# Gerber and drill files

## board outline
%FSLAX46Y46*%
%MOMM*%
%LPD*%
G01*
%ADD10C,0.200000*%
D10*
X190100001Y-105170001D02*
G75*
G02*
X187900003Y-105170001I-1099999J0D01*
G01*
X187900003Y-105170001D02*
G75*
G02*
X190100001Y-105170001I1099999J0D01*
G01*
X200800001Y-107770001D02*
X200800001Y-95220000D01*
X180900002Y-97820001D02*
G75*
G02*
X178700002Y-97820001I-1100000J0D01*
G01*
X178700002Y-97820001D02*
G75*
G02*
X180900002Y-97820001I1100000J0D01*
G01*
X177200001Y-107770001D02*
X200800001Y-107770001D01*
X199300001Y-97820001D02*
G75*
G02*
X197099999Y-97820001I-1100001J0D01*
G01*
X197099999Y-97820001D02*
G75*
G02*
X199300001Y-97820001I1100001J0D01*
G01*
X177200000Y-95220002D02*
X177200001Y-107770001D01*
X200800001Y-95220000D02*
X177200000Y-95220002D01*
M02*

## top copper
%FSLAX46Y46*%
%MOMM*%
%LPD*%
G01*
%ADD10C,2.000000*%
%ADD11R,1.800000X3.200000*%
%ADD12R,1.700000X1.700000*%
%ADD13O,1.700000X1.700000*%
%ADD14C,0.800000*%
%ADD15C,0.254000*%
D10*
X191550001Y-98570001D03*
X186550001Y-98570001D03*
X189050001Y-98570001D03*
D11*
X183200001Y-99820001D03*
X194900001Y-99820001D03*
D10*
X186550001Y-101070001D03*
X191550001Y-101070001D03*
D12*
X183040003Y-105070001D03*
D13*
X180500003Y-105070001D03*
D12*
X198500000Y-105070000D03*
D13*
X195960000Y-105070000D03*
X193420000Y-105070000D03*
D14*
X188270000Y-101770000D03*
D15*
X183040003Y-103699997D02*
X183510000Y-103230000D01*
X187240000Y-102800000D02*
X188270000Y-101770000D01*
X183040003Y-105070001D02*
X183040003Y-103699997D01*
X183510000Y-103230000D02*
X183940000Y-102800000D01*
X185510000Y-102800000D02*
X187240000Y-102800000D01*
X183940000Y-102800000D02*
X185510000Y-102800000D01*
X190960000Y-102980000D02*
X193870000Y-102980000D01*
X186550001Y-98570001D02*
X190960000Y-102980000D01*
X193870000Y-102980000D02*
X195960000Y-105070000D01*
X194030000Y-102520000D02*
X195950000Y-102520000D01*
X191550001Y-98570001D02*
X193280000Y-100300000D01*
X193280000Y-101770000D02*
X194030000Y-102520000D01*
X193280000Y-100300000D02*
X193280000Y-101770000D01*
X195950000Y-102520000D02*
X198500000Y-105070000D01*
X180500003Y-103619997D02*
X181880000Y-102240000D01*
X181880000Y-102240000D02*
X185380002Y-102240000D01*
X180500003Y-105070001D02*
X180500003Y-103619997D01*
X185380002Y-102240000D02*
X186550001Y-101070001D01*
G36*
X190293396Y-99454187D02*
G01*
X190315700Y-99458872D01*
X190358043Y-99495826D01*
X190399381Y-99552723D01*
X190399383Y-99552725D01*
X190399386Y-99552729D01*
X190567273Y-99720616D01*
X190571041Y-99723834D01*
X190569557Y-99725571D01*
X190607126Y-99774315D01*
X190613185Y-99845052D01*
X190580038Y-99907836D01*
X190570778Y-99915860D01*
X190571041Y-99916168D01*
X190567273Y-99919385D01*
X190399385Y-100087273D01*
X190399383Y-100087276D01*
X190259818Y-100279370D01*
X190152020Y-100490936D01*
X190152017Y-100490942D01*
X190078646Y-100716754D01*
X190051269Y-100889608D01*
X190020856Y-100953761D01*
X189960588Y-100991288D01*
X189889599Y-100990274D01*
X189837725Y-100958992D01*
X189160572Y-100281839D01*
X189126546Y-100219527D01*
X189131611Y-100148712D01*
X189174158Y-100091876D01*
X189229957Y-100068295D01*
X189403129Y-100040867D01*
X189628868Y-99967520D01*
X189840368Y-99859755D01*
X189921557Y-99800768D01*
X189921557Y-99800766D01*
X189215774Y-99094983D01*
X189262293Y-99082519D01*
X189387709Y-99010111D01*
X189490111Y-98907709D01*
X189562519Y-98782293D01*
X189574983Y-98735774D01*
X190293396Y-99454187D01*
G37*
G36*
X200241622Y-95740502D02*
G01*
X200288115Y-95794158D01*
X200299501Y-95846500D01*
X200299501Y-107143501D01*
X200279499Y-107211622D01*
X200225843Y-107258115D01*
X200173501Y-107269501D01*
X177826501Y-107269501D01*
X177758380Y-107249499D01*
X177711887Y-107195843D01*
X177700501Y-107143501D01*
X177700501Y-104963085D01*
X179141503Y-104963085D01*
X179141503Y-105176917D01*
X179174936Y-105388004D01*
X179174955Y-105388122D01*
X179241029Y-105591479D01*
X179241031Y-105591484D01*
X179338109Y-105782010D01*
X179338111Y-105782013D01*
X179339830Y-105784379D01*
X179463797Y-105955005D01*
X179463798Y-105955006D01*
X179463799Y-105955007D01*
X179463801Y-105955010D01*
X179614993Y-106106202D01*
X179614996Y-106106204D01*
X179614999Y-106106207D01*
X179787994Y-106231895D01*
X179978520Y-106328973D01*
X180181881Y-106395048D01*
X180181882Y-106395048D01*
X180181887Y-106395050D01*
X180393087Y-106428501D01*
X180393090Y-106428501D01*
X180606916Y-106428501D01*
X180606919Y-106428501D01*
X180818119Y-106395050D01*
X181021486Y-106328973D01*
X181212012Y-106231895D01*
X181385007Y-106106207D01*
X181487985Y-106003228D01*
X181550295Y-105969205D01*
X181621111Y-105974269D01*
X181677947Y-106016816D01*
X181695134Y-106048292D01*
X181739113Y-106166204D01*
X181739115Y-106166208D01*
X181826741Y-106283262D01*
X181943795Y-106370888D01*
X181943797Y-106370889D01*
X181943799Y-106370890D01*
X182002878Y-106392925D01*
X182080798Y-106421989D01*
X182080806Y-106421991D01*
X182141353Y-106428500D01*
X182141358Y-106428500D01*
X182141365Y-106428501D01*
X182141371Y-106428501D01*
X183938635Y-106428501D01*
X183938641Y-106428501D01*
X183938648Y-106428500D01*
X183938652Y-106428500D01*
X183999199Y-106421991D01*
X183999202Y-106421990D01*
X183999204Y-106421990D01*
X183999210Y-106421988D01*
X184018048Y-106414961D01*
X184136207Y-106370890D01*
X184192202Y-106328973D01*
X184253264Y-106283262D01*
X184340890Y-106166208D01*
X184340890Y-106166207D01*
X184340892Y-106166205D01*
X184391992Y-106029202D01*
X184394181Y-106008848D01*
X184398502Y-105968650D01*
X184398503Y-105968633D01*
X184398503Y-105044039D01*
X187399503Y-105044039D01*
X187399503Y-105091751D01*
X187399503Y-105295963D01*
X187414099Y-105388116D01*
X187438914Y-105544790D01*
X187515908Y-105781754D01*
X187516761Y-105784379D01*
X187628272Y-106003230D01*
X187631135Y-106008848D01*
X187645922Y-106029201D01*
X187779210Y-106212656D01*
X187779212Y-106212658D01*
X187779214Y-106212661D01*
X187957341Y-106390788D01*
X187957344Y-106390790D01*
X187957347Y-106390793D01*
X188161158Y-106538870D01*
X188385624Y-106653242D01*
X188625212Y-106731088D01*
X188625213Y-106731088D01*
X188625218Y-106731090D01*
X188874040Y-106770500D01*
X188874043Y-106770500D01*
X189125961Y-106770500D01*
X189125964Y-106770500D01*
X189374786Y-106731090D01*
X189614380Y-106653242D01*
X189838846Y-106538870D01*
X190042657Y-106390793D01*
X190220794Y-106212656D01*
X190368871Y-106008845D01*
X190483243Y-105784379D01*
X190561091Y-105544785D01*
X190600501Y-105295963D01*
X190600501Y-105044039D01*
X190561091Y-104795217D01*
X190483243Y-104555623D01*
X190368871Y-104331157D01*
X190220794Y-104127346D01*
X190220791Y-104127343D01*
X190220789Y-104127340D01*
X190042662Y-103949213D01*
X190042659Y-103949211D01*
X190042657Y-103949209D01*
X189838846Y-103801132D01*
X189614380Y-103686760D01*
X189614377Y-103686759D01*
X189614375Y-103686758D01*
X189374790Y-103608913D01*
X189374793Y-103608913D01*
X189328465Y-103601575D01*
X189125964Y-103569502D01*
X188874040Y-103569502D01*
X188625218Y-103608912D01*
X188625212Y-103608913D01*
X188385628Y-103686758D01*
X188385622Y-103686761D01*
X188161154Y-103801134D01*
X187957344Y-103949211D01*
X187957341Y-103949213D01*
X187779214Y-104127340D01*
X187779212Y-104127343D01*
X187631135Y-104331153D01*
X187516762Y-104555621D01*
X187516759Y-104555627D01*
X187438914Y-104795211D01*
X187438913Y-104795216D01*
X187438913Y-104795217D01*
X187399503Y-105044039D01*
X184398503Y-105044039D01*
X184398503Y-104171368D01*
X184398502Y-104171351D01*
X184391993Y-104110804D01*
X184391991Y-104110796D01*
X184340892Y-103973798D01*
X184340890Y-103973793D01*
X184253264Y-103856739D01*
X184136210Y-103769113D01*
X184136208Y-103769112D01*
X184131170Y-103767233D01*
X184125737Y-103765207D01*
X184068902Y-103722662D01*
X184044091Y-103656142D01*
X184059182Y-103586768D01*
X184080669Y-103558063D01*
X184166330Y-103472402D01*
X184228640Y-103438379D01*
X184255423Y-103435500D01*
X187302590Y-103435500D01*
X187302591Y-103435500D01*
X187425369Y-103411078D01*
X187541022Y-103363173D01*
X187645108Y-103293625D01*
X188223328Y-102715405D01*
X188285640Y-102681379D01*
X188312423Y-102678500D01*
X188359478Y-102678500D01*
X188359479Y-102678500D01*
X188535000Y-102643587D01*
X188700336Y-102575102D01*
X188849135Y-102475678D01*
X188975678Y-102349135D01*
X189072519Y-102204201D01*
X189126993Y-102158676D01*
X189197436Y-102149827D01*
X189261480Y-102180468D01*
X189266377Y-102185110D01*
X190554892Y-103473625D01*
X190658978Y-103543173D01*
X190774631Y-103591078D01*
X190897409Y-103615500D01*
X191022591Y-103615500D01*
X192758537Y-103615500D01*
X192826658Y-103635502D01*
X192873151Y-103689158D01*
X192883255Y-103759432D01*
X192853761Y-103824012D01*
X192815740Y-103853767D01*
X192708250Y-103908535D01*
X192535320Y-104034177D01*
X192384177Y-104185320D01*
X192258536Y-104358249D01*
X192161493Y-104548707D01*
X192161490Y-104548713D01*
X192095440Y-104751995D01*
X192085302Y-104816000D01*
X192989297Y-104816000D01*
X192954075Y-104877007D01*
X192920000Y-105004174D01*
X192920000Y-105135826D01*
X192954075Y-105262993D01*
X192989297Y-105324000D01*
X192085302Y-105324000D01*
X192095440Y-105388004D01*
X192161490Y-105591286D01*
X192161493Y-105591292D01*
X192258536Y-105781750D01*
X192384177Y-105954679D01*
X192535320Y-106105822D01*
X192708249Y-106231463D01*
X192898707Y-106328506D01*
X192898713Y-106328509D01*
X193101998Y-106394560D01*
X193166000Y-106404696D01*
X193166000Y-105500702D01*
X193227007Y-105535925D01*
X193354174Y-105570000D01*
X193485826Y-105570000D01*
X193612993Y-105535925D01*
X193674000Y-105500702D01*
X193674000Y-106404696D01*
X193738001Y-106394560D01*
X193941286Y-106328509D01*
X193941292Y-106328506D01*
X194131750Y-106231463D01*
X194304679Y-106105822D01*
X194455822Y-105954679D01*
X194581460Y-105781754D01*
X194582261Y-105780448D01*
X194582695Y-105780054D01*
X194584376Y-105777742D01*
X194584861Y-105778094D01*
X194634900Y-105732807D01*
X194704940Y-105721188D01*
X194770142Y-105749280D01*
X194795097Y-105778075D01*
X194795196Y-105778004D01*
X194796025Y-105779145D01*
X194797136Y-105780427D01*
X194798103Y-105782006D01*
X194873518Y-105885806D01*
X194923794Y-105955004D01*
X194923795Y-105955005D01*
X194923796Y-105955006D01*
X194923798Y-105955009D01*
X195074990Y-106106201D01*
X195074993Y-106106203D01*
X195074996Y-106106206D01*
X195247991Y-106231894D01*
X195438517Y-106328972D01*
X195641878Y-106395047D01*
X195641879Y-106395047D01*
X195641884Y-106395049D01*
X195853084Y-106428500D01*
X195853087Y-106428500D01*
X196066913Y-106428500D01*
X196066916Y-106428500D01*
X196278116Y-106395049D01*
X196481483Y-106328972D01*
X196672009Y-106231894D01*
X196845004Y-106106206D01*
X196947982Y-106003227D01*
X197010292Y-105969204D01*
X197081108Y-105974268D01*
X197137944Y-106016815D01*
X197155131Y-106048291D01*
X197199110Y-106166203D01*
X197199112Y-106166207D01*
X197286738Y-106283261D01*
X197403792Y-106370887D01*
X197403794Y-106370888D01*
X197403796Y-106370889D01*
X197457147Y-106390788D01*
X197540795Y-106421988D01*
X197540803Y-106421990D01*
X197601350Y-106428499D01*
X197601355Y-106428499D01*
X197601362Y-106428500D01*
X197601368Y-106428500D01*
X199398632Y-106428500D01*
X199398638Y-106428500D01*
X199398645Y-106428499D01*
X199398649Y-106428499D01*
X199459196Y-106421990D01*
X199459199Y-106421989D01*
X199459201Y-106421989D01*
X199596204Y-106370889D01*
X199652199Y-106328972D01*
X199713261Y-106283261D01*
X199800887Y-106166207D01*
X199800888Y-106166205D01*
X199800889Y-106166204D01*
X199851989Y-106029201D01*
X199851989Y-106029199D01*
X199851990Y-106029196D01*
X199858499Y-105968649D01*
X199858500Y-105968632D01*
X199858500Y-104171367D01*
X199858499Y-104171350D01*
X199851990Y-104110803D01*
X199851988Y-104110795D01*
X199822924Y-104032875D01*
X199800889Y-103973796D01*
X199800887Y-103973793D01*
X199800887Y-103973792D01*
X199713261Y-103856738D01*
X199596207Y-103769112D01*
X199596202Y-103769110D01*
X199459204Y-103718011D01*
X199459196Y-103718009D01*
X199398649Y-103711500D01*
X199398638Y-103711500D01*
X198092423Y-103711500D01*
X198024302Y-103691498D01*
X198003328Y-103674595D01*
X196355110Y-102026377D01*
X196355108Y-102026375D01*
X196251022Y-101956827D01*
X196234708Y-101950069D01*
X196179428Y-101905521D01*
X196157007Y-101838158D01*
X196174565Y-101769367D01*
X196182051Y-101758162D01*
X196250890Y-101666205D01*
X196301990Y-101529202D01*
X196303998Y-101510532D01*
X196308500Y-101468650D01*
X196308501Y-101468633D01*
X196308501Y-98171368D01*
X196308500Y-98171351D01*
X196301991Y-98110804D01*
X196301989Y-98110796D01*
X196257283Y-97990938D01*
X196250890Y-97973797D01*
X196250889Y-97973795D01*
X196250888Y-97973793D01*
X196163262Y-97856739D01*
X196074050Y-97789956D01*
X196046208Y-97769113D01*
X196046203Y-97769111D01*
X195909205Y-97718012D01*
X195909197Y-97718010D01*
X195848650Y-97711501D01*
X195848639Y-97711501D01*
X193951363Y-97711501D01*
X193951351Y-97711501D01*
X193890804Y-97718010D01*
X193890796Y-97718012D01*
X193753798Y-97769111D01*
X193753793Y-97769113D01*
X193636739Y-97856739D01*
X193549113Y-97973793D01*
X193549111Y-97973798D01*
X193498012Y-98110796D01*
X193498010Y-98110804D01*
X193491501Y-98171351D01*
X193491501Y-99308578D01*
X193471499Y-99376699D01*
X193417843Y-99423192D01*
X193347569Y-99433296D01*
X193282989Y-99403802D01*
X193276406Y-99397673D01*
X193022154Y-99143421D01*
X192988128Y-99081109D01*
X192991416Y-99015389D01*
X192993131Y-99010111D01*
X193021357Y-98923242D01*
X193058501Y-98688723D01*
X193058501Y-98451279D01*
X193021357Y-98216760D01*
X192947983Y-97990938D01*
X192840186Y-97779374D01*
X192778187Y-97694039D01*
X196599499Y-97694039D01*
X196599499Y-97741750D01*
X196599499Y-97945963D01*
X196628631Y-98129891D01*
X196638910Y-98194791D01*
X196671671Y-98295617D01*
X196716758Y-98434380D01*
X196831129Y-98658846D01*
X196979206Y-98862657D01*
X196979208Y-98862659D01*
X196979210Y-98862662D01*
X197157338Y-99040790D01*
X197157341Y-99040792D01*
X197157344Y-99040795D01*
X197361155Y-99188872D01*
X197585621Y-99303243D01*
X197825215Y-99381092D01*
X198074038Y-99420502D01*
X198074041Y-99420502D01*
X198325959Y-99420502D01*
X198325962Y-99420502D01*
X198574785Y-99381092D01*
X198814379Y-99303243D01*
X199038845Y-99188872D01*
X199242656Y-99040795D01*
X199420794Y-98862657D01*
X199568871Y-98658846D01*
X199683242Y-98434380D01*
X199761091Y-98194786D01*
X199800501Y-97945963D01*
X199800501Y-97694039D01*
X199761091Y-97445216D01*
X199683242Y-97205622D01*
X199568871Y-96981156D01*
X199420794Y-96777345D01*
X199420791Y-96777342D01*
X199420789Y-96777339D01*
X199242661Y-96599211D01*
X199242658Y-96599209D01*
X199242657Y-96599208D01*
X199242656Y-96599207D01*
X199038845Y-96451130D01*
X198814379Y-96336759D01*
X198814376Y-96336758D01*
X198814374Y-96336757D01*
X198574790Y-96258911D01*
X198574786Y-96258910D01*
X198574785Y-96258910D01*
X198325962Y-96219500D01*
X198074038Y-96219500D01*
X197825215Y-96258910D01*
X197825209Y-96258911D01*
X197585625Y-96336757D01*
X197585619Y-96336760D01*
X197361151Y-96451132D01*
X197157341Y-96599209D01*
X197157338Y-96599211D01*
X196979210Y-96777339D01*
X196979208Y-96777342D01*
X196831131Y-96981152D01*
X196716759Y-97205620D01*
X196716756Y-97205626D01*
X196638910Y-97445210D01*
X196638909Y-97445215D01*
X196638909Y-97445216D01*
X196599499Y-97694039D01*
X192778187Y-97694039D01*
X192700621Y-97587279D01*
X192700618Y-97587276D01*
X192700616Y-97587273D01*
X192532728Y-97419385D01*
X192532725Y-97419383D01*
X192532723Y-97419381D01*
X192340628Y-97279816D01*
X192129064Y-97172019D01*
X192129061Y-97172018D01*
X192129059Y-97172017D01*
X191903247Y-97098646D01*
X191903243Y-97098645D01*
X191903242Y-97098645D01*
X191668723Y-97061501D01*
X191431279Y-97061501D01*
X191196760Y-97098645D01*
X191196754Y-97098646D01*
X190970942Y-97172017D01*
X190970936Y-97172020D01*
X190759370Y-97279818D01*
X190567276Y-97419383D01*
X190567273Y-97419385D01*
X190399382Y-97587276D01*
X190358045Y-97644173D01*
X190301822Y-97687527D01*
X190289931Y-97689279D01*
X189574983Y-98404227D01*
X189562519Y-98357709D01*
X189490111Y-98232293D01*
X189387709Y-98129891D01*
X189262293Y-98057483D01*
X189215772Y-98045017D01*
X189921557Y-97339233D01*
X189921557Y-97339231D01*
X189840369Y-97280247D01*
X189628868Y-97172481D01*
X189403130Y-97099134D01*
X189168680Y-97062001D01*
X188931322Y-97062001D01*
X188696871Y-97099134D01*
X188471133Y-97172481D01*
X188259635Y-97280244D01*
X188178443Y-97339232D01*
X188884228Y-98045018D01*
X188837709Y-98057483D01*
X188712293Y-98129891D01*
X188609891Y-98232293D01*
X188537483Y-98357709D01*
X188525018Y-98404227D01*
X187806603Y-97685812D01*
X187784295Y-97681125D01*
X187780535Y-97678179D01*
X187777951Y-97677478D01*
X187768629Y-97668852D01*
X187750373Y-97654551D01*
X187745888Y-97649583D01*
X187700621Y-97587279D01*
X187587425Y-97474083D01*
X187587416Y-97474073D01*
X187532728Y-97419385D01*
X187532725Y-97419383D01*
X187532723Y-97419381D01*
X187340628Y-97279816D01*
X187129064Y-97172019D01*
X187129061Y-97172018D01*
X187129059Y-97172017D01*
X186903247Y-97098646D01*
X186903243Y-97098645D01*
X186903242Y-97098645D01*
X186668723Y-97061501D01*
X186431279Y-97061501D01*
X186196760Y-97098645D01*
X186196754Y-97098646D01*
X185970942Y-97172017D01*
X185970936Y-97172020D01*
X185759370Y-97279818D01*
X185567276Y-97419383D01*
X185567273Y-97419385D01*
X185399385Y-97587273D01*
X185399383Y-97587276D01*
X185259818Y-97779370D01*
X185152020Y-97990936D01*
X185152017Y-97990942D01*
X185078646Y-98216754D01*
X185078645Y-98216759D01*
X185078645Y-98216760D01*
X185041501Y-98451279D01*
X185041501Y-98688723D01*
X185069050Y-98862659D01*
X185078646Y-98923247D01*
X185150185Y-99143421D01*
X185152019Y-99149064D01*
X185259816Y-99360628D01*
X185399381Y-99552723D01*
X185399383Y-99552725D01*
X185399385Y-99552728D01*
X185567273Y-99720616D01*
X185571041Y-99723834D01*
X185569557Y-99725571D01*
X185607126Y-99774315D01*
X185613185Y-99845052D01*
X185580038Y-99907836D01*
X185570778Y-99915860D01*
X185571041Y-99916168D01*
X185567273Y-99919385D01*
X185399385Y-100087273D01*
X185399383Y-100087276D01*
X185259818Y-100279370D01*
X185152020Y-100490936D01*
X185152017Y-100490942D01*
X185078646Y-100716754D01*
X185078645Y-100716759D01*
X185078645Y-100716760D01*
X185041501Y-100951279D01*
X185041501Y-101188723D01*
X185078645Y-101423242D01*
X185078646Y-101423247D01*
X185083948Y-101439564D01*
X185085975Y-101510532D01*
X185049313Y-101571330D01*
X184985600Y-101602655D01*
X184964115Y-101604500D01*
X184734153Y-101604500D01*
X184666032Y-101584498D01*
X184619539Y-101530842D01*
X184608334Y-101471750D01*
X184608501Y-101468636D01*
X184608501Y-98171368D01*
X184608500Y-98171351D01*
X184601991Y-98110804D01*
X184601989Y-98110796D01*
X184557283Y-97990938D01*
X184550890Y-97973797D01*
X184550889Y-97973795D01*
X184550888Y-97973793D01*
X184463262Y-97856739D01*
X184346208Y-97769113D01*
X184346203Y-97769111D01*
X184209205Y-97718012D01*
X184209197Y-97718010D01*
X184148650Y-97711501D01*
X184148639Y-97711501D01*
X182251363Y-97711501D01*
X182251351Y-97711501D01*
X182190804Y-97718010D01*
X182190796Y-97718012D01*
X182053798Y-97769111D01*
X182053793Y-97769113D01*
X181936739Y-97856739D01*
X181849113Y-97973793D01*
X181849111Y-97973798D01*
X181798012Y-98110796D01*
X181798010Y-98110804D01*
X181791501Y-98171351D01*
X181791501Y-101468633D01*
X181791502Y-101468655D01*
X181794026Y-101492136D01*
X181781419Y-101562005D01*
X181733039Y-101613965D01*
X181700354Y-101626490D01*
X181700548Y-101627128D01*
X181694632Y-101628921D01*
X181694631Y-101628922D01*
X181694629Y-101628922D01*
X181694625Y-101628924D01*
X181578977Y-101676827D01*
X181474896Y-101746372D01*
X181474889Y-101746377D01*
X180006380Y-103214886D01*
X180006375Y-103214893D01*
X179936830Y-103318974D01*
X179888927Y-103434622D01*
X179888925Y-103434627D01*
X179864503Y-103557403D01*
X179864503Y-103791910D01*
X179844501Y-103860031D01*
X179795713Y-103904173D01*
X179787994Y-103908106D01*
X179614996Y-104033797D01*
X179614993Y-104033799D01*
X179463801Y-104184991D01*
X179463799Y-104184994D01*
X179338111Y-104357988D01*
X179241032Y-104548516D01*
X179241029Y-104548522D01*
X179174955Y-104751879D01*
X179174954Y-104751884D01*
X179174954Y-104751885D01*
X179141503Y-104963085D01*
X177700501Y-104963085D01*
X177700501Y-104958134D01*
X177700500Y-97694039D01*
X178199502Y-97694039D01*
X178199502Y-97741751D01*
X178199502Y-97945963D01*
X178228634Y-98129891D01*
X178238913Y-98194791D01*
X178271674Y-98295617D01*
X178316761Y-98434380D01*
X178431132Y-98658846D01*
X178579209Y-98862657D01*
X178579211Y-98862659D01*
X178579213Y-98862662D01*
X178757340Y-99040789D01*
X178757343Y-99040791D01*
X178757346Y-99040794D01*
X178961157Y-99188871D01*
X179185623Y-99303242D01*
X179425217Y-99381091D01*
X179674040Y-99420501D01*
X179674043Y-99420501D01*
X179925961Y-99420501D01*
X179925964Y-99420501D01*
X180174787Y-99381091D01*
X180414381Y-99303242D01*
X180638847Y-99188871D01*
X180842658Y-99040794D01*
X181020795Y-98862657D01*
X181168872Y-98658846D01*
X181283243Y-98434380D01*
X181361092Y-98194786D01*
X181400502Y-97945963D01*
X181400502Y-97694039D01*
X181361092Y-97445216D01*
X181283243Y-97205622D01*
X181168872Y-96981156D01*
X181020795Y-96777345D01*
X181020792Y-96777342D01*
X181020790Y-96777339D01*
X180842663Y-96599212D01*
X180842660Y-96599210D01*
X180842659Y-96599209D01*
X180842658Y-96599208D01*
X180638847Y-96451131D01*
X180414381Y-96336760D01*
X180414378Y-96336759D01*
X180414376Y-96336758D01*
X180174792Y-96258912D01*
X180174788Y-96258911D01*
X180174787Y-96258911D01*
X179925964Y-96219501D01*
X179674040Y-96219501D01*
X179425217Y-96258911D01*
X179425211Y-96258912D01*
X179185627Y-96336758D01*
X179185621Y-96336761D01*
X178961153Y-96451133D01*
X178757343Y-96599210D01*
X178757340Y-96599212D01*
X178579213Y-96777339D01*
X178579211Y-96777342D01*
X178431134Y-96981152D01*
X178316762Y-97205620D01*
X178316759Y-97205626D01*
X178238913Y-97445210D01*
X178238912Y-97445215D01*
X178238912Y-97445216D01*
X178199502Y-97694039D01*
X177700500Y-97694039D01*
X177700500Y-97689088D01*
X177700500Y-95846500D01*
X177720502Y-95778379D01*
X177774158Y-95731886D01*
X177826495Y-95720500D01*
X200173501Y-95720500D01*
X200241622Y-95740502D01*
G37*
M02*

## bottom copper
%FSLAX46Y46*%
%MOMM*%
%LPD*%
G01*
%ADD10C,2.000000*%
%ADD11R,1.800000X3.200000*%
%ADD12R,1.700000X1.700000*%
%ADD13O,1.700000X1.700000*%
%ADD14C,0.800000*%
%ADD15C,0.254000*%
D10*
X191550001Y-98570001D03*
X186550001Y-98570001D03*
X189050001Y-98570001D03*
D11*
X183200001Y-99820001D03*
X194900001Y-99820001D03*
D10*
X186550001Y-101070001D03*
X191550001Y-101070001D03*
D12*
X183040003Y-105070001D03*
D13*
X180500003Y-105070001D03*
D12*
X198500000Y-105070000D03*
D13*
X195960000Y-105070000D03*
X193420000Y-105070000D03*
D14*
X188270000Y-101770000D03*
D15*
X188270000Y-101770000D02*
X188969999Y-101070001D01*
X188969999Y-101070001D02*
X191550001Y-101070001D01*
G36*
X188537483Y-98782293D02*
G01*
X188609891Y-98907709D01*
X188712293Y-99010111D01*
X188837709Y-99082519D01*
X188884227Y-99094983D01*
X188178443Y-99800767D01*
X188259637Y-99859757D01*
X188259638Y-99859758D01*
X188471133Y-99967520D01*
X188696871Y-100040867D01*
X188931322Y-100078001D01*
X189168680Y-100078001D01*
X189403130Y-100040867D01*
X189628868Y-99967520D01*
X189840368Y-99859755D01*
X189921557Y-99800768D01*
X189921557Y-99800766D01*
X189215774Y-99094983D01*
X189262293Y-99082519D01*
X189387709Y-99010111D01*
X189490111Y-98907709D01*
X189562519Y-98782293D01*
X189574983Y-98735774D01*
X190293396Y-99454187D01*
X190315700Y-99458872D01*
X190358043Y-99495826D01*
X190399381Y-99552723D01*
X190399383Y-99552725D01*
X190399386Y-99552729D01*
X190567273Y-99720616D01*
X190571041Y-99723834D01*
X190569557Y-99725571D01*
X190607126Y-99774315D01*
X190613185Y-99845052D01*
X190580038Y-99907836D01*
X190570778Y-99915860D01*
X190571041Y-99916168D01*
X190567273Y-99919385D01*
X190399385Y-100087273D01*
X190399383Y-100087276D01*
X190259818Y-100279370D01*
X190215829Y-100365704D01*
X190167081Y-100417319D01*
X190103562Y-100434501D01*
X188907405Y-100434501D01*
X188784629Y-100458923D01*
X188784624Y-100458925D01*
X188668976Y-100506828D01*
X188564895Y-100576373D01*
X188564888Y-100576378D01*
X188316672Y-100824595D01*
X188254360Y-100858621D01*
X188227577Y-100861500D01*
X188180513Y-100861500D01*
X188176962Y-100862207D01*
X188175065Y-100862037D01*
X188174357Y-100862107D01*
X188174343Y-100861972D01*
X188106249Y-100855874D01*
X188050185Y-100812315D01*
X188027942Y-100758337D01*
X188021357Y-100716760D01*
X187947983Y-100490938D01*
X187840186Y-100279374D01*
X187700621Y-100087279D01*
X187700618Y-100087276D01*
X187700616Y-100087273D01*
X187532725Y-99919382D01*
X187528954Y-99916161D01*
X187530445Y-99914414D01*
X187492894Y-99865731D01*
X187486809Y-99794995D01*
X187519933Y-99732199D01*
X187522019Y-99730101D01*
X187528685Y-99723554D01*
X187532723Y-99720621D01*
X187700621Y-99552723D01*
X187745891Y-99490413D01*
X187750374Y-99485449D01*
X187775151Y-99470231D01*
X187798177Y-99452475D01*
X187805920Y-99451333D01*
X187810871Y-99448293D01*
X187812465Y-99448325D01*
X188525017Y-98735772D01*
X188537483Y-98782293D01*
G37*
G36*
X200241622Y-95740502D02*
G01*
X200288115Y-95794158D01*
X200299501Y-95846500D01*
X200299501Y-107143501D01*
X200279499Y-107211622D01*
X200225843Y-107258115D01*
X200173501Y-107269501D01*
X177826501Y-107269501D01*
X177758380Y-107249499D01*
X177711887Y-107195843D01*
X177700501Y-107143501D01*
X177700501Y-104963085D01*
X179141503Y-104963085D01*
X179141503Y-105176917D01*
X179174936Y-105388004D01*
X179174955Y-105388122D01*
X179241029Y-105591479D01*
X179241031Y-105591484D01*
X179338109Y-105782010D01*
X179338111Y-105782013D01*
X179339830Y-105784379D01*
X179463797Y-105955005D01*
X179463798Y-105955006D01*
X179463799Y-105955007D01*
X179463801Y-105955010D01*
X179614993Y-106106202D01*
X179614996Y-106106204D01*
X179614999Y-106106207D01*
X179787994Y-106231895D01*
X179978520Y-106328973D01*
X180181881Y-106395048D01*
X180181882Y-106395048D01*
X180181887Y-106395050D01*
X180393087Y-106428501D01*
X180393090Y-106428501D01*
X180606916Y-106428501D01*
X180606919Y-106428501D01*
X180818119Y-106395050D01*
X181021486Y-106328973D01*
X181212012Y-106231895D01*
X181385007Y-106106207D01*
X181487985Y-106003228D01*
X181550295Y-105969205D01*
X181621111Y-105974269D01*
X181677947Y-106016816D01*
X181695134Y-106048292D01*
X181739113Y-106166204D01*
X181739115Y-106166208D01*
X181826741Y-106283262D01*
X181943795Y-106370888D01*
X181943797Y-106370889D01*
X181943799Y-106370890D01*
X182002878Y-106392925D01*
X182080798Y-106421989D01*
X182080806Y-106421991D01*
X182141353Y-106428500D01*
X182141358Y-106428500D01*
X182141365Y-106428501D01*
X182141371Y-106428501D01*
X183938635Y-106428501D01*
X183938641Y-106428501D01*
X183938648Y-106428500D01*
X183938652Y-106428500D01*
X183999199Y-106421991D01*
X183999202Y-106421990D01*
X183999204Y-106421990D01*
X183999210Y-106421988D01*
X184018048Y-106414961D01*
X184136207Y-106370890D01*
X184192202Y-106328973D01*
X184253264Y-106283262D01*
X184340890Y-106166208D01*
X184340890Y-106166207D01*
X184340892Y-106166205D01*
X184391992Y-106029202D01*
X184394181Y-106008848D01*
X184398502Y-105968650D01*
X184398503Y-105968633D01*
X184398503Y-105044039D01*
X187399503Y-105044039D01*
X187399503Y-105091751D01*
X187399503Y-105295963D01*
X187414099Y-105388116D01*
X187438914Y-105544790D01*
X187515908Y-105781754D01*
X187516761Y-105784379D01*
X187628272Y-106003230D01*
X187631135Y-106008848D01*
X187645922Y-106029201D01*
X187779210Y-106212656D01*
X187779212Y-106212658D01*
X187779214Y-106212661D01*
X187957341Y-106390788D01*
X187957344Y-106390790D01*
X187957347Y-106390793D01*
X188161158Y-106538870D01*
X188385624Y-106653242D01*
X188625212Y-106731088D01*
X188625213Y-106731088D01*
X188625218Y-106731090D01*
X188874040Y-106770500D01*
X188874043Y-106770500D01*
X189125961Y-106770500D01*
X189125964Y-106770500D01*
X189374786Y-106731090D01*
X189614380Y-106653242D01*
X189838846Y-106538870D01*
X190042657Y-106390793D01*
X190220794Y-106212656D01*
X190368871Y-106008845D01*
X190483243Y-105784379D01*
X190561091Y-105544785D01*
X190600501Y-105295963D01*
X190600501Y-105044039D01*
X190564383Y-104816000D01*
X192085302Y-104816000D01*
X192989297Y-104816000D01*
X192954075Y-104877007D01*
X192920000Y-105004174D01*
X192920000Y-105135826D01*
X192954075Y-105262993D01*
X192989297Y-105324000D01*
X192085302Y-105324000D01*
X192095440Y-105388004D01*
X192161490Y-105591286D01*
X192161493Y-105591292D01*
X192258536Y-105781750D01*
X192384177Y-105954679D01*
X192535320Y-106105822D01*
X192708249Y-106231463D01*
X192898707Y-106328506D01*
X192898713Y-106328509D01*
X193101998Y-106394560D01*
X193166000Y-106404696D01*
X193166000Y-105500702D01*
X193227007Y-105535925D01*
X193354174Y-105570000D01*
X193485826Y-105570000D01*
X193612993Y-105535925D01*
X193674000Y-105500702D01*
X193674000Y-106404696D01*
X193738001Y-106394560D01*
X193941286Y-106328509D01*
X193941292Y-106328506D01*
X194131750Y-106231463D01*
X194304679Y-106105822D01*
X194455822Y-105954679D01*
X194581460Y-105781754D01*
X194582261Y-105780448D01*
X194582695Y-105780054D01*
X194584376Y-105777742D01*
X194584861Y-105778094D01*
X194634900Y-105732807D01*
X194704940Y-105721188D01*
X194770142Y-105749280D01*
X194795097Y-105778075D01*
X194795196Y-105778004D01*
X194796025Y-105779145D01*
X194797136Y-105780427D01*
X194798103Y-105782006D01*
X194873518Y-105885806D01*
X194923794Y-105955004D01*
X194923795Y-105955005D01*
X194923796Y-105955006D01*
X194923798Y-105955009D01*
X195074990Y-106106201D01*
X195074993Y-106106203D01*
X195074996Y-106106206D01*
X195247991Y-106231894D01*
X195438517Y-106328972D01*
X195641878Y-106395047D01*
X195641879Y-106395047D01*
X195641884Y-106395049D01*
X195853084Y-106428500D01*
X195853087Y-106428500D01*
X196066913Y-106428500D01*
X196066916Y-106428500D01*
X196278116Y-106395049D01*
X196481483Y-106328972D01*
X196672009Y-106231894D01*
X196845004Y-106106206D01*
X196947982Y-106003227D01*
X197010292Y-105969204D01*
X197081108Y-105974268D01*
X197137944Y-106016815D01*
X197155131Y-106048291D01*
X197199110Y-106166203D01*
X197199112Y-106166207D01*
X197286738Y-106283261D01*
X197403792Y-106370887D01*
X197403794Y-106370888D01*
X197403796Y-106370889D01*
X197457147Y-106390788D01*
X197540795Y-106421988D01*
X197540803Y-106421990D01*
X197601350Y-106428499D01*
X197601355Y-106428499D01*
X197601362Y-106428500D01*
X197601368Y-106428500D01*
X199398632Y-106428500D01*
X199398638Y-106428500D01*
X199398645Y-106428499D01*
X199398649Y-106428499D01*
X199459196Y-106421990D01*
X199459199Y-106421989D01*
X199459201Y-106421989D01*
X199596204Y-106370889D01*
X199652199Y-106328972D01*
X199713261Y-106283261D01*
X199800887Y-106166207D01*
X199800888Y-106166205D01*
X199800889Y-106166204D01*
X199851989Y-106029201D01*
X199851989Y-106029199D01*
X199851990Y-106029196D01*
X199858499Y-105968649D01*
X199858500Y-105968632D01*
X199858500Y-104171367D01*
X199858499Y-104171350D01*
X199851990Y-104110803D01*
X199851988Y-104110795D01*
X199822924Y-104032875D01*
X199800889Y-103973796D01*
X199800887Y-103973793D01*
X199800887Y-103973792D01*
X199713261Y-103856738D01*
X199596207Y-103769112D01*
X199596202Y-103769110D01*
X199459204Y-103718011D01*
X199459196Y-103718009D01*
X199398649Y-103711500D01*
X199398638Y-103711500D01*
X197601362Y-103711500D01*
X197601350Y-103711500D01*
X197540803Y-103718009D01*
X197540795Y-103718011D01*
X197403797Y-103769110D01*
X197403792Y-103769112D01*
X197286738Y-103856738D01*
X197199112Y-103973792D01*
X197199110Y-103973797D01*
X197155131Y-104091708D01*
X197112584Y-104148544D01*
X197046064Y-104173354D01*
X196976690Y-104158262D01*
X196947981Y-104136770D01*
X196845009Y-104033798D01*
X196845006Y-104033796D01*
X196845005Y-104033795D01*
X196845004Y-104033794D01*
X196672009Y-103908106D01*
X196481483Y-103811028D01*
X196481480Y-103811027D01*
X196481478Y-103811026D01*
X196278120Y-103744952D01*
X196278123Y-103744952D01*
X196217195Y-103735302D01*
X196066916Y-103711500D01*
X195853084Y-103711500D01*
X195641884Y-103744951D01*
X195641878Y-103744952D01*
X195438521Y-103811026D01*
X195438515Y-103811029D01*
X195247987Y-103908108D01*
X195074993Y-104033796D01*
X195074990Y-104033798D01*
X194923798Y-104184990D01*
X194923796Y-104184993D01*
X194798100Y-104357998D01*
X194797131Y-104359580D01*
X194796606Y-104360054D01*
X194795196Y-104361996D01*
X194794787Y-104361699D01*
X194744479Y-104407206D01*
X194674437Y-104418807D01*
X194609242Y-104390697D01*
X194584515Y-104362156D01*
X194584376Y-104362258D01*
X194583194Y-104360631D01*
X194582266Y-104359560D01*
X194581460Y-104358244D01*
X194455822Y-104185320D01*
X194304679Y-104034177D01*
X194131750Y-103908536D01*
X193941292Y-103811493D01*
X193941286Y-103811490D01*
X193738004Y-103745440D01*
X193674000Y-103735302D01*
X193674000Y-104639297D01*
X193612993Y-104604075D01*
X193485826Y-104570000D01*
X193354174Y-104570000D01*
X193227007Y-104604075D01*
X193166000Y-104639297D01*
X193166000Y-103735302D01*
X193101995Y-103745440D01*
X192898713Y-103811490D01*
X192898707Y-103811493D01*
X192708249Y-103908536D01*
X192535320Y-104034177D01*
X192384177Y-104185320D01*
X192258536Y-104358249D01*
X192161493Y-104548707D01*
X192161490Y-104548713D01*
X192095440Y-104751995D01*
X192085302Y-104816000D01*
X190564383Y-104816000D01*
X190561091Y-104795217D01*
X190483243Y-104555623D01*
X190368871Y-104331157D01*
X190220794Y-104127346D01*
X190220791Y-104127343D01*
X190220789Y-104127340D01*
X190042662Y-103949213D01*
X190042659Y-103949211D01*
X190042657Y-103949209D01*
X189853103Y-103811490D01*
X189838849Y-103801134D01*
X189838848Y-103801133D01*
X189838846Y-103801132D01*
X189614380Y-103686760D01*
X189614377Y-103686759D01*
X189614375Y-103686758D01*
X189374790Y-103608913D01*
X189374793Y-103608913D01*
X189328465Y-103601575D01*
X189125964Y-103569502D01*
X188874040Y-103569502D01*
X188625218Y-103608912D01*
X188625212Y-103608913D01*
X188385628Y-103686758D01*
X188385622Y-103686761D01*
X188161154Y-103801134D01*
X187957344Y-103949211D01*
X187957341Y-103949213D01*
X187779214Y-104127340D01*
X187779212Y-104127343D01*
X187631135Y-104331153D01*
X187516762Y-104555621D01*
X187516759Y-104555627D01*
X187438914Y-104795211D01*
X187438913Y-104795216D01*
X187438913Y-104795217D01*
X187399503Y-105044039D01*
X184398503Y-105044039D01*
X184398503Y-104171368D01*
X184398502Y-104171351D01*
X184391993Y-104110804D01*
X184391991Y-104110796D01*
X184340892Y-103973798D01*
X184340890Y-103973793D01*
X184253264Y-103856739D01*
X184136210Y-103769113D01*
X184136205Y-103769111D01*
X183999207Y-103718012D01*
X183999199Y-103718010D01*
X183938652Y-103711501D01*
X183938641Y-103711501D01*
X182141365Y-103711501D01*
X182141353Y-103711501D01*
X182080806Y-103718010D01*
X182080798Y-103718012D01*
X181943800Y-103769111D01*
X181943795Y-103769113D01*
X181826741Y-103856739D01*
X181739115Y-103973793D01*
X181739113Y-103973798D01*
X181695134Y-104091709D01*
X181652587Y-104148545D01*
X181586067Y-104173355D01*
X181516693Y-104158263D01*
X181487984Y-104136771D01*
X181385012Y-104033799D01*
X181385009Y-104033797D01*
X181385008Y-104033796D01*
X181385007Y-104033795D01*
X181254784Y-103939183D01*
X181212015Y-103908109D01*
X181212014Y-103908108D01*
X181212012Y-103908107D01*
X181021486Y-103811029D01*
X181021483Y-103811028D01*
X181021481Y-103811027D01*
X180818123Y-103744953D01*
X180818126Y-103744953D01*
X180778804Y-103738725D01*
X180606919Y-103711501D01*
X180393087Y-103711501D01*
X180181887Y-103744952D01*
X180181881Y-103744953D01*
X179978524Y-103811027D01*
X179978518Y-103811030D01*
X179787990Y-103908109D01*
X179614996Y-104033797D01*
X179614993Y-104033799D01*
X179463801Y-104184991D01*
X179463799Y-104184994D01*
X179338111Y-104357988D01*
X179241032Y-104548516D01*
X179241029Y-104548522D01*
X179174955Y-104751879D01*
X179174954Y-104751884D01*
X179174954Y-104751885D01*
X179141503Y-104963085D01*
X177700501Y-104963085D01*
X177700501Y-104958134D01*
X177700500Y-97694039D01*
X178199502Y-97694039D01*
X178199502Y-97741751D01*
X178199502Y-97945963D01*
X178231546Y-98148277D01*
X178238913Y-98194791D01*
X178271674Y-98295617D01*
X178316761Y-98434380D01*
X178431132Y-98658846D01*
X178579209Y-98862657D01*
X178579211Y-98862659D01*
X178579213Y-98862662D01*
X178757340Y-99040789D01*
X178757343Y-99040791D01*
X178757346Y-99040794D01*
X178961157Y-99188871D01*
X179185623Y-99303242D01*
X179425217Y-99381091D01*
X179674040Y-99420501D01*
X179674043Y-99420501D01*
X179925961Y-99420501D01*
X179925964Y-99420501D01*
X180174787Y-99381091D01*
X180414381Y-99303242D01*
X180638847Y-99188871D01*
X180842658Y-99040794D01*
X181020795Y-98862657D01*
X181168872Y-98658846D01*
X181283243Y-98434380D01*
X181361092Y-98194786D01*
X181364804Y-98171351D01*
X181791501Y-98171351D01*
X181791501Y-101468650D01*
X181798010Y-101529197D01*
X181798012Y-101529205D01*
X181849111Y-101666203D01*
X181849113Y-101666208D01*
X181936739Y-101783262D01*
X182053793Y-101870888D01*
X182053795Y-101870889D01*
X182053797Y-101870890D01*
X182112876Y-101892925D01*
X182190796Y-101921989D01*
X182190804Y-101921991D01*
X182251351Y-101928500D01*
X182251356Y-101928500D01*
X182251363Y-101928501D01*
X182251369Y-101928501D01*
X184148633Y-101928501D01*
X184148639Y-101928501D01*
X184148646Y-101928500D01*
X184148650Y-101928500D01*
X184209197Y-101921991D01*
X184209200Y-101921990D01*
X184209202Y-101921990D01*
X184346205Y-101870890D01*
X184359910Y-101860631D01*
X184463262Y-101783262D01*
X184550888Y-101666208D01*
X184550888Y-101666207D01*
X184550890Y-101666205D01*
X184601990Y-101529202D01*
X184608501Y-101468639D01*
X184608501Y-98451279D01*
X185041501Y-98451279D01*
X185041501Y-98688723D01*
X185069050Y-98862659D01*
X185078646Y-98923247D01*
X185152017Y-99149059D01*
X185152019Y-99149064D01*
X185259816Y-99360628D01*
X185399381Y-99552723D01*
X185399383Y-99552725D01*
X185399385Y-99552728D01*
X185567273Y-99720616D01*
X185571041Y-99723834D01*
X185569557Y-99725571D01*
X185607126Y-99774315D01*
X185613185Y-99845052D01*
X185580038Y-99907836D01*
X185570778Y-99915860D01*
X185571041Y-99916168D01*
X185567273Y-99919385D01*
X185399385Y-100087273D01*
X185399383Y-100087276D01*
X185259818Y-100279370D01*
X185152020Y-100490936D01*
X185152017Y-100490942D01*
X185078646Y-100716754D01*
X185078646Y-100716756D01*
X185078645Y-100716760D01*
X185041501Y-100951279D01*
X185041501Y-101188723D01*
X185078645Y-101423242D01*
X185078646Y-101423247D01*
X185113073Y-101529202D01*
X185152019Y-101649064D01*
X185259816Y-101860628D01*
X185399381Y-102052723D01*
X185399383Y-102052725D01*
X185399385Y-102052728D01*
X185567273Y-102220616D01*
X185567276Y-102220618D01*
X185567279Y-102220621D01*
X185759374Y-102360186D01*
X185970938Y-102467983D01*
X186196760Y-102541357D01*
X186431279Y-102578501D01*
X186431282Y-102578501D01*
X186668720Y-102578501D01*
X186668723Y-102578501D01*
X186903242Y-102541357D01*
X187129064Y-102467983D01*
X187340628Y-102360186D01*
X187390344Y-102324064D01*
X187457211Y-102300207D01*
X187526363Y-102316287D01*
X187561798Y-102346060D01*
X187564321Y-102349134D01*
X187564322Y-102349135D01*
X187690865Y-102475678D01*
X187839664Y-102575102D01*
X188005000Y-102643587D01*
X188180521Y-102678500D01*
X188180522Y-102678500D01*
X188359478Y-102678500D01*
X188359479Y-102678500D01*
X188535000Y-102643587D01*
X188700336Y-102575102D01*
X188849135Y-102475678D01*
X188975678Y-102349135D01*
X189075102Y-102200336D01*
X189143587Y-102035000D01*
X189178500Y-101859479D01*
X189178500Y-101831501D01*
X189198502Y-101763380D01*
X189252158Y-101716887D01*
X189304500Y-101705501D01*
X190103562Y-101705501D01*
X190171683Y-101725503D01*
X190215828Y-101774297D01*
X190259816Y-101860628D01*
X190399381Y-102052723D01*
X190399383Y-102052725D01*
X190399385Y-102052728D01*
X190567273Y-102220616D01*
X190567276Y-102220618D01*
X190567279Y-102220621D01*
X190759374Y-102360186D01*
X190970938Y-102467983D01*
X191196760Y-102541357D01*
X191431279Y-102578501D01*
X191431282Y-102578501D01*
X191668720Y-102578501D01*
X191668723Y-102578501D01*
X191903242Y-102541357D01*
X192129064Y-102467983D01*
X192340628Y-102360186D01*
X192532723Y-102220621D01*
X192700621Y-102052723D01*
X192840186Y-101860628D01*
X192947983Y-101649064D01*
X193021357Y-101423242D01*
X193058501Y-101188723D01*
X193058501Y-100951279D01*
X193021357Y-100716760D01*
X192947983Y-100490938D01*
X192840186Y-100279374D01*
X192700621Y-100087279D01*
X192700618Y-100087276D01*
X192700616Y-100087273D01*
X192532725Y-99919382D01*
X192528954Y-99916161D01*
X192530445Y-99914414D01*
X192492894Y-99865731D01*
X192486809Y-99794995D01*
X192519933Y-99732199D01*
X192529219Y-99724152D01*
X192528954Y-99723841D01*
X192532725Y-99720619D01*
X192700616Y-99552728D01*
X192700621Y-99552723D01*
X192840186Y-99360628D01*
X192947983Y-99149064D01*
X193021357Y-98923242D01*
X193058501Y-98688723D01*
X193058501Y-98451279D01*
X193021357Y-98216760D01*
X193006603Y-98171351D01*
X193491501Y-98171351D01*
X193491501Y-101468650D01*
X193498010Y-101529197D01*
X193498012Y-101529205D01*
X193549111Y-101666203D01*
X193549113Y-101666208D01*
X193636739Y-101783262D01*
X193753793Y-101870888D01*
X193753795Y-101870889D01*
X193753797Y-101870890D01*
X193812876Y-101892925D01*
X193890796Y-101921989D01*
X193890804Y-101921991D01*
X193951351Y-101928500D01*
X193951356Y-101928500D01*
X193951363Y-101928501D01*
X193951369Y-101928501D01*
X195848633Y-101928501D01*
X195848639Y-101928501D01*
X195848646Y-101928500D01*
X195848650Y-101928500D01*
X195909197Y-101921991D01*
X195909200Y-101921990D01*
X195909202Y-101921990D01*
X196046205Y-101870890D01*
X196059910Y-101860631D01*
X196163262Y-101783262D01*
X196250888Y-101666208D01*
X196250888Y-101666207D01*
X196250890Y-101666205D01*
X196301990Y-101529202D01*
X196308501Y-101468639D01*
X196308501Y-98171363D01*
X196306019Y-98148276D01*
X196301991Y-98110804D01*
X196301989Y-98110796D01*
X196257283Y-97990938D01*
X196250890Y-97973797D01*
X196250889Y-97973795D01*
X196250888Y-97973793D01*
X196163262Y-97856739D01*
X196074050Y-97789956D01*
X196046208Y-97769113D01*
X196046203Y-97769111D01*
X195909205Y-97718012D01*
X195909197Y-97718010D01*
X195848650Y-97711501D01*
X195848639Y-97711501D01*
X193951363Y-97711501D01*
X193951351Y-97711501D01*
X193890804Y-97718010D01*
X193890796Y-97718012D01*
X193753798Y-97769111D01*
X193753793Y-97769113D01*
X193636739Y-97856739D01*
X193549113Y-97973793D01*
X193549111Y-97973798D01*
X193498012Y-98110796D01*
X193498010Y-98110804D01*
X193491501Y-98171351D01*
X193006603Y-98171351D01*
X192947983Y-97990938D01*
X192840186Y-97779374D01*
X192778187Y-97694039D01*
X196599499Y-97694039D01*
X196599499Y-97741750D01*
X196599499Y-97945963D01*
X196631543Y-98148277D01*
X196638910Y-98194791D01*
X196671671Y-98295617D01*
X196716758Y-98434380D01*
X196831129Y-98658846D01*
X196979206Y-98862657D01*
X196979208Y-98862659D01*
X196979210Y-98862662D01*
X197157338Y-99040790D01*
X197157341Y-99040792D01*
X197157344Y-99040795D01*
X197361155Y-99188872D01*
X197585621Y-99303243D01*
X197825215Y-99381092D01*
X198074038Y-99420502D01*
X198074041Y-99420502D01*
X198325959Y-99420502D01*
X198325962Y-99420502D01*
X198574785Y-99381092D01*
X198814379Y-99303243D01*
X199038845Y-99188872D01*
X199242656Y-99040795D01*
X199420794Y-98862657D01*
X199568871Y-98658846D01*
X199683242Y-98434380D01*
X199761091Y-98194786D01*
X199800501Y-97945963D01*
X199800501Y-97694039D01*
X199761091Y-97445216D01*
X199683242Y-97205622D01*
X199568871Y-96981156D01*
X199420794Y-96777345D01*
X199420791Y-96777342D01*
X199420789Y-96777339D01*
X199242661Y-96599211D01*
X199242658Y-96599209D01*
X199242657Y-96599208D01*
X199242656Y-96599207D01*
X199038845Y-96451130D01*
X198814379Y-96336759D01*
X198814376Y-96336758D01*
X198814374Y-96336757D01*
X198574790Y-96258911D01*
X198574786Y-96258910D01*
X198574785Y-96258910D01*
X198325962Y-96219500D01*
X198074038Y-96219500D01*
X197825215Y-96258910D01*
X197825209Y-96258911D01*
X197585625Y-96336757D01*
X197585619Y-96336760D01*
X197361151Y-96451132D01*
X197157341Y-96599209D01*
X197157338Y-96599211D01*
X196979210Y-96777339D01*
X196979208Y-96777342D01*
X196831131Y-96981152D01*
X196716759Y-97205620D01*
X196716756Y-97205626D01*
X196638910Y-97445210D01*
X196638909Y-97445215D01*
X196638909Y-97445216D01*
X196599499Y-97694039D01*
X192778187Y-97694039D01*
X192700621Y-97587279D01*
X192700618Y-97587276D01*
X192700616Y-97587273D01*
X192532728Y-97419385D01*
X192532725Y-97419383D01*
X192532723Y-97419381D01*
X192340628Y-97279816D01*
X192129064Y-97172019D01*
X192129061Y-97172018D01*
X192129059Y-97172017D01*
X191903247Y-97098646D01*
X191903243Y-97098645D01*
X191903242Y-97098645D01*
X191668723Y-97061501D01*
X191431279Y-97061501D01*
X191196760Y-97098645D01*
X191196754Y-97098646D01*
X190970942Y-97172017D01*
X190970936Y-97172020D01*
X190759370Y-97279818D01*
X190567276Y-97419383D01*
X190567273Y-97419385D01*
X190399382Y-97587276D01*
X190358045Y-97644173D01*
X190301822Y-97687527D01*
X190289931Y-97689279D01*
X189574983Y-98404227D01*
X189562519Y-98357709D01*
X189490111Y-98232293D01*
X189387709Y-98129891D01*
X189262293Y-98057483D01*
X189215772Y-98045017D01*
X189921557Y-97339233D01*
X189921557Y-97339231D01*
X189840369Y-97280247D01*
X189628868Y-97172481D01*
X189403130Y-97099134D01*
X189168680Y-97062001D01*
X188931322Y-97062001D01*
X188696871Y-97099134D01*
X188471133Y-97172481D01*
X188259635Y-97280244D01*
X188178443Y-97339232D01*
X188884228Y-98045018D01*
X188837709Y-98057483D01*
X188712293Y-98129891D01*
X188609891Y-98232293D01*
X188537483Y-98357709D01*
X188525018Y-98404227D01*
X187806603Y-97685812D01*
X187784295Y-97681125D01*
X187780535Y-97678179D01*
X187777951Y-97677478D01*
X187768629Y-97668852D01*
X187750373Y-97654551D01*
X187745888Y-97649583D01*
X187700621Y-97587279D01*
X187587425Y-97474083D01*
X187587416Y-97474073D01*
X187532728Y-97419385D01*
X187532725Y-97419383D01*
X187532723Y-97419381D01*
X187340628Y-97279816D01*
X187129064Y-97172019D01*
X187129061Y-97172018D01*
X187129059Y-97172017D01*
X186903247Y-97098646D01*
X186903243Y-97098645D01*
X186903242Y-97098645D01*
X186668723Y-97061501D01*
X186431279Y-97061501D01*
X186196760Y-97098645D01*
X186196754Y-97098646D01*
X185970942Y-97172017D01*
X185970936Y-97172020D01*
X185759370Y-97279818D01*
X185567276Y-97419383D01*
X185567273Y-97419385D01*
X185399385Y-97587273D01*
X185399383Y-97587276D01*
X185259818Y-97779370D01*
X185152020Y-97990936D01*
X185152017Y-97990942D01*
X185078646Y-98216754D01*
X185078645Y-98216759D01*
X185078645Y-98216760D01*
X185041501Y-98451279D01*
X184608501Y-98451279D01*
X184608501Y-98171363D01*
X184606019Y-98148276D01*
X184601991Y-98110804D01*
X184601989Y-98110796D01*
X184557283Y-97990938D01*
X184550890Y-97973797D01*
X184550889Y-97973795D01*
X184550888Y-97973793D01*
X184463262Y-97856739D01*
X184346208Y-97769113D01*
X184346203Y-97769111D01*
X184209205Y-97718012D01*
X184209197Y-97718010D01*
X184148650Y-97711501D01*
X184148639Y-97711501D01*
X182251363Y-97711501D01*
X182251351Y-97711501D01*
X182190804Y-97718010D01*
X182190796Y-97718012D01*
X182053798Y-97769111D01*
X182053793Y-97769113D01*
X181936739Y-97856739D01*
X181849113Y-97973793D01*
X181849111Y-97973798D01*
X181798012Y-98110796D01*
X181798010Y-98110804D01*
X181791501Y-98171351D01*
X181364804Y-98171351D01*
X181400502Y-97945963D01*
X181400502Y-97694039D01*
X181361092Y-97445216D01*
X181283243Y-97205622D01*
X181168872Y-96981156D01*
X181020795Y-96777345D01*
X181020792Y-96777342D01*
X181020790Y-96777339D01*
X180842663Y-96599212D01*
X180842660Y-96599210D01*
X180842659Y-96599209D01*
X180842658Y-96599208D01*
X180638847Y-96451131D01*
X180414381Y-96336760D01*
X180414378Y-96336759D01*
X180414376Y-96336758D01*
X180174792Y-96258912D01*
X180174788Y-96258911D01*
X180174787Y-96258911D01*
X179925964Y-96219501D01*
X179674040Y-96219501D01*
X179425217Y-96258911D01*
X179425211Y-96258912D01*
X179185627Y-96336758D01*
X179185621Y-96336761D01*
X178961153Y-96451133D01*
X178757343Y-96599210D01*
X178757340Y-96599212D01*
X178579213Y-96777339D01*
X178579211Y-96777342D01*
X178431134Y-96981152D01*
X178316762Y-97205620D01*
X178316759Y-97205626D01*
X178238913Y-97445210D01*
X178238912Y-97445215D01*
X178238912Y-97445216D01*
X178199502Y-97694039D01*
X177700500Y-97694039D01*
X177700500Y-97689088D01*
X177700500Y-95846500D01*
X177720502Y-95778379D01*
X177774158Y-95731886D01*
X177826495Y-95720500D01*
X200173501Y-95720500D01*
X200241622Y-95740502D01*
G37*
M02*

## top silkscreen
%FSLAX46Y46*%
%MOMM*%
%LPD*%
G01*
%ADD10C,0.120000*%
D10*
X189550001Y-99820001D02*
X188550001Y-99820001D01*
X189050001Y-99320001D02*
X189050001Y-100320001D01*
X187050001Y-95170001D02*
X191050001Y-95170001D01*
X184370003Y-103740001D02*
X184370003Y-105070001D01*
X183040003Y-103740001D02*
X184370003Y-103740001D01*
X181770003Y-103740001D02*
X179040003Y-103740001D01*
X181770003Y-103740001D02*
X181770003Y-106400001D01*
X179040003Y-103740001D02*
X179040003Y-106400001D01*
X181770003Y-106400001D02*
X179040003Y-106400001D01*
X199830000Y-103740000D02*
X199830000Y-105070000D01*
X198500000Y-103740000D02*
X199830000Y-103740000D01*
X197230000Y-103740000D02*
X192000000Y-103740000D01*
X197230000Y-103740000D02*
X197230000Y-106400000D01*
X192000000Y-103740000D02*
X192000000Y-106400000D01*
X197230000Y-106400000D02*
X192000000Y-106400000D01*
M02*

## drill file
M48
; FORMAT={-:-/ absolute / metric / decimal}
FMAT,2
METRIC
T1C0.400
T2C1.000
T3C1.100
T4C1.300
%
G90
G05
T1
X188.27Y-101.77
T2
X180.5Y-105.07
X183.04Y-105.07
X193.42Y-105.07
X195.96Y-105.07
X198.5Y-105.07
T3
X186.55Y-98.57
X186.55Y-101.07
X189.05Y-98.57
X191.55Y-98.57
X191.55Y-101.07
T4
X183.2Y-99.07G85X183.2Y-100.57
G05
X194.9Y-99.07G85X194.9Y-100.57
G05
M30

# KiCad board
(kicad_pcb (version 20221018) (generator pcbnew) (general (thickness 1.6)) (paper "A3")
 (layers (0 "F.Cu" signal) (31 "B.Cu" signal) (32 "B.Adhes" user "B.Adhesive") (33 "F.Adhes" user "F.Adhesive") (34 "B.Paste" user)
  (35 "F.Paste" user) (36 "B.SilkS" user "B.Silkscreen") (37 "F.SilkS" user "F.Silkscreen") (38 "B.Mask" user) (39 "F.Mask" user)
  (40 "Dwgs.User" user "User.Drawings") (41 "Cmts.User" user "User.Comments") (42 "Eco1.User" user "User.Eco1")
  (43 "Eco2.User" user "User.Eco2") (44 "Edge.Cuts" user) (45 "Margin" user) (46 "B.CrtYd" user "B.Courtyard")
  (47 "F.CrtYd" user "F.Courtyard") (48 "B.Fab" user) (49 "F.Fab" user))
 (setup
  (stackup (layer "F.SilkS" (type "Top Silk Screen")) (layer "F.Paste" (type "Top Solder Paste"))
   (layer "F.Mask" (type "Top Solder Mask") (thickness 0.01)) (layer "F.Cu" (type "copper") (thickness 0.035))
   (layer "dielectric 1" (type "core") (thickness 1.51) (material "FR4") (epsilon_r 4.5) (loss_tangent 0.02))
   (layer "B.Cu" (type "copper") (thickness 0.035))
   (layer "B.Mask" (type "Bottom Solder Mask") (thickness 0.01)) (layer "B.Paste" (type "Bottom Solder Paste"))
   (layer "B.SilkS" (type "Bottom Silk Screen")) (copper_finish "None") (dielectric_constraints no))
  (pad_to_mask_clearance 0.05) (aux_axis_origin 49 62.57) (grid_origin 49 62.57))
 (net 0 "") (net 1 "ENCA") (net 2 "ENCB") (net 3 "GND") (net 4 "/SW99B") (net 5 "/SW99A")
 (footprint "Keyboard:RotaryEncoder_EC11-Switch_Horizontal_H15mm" (layer "F.Cu") (at 189.050001 99.820001 90)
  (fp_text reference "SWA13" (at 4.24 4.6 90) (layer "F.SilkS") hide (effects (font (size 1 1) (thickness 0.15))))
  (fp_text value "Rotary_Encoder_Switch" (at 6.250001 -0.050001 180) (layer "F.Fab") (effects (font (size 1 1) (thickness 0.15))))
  (fp_line (start 0 0.5) (end 0 -0.5) (stroke (width 0.12) (type solid)) (layer "F.SilkS"))
  (fp_line (start 0.5 0) (end -0.5 0) (stroke (width 0.12) (type solid)) (layer "F.SilkS"))
  (fp_line (start 4.65 -2) (end 4.65 2) (stroke (width 0.12) (type solid)) (layer "F.SilkS"))
  (pad "A" thru_hole circle (at 1.25 2.5 270) (size 2 2) (drill 1.1) (layers "*.Cu" "*.Mask") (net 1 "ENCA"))
  (pad "B" thru_hole circle (at 1.25 -2.5 270) (size 2 2) (drill 1.1) (layers "*.Cu" "*.Mask") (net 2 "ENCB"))
  (pad "C" thru_hole circle (at 1.25 0 270) (size 2 2) (drill 1.1) (layers "*.Cu" "*.Mask") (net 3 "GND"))
  (pad "MP" thru_hole rect (at 0 -5.85 270) (size 3.2 1.8) (drill oval 2.8 1.3) (layers "*.Cu" "*.Mask"))
  (pad "MP" thru_hole rect (at 0 5.85 270) (size 3.2 1.8) (drill oval 2.8 1.3) (layers "*.Cu" "*.Mask"))
  (pad "S1" thru_hole circle (at -1.25 -2.5 270) (size 2 2) (drill 1.1) (layers "*.Cu" "*.Mask") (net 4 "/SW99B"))
  (pad "S2" thru_hole circle (at -1.25 2.5 270) (size 2 2) (drill 1.1) (layers "*.Cu" "*.Mask") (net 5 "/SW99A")))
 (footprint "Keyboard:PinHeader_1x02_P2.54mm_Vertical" (layer "F.Cu") (at 183.040003 105.070001 -90)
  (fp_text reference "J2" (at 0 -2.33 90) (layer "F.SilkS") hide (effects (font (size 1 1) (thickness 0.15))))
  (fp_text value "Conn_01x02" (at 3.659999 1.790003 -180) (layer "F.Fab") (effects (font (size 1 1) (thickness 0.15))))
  (fp_line (start -1.33 -1.33) (end 0 -1.33) (stroke (width 0.12) (type solid)) (layer "F.SilkS"))
  (fp_line (start -1.33 0) (end -1.33 -1.33) (stroke (width 0.12) (type solid)) (layer "F.SilkS"))
  (fp_line (start -1.33 1.27) (end -1.33 4) (stroke (width 0.12) (type solid)) (layer "F.SilkS"))
  (fp_line (start -1.33 1.27) (end 1.33 1.27) (stroke (width 0.12) (type solid)) (layer "F.SilkS"))
  (fp_line (start -1.33 4) (end 1.33 4) (stroke (width 0.12) (type solid)) (layer "F.SilkS"))
  (fp_line (start 1.33 1.27) (end 1.33 4) (stroke (width 0.12) (type solid)) (layer "F.SilkS"))
  (pad "1" thru_hole rect (at 0 0 270) (size 1.7 1.7) (drill 1) (layers "*.Cu" "*.Mask") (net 5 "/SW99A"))
  (pad "2" thru_hole oval (at 0 2.54 270) (size 1.7 1.7) (drill 1) (layers "*.Cu" "*.Mask") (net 4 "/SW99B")))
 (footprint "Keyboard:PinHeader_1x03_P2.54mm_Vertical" (layer "F.Cu") (at 198.5 105.07 -90)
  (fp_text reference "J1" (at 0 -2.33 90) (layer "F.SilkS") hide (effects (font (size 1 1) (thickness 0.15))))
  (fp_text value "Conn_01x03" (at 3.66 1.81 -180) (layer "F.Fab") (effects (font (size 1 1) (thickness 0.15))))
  (fp_line (start -1.33 -1.33) (end 0 -1.33) (stroke (width 0.12) (type solid)) (layer "F.SilkS"))
  (fp_line (start -1.33 0) (end -1.33 -1.33) (stroke (width 0.12) (type solid)) (layer "F.SilkS"))
  (fp_line (start -1.33 1.27) (end -1.33 6.5) (stroke (width 0.12) (type solid)) (layer "F.SilkS"))
  (fp_line (start -1.33 1.27) (end 1.33 1.27) (stroke (width 0.12) (type solid)) (layer "F.SilkS"))
  (fp_line (start -1.33 6.5) (end 1.33 6.5) (stroke (width 0.12) (type solid)) (layer "F.SilkS"))
  (fp_line (start 1.33 1.27) (end 1.33 6.5) (stroke (width 0.12) (type solid)) (layer "F.SilkS"))
  (pad "1" thru_hole rect (at 0 0 270) (size 1.7 1.7) (drill 1) (layers "*.Cu" "*.Mask") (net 1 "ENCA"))
  (pad "2" thru_hole oval (at 0 2.54 270) (size 1.7 1.7) (drill 1) (layers "*.Cu" "*.Mask") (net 2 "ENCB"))
  (pad "3" thru_hole oval (at 0 5.08 270) (size 1.7 1.7) (drill 1) (layers "*.Cu" "*.Mask") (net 3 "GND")))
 (gr_circle (center 189.000002 105.170001) (end 190.100001 105.170001) (stroke (width 0.2) (type solid)) (fill none) (layer "Edge.Cuts"))
 (gr_line (start 200.800001 107.770001) (end 200.800001 95.22) (stroke (width 0.2) (type solid)) (layer "Edge.Cuts"))
 (gr_circle (center 179.800002 97.820001) (end 180.900002 97.820001) (stroke (width 0.2) (type solid)) (fill none) (layer "Edge.Cuts"))
 (gr_line (start 177.200001 107.770001) (end 200.800001 107.770001) (stroke (width 0.2) (type solid)) (layer "Edge.Cuts"))
 (gr_circle (center 198.2 97.820001) (end 199.300001 97.820001) (stroke (width 0.2) (type solid)) (fill none) (layer "Edge.Cuts"))
 (gr_line (start 177.2 95.220002) (end 177.200001 107.770001) (stroke (width 0.2) (type solid)) (layer "Edge.Cuts"))
 (gr_line (start 200.800001 95.22) (end 177.2 95.220002) (stroke (width 0.2) (type solid)) (layer "Edge.Cuts"))
 (segment (start 183.040003 103.699997) (end 183.51 103.23) (width 0.254) (layer "F.Cu") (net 5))
 (segment (start 187.24 102.8) (end 188.27 101.77) (width 0.254) (layer "F.Cu") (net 5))
 (segment (start 183.040003 105.070001) (end 183.040003 103.699997) (width 0.254) (layer "F.Cu") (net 5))
 (segment (start 183.51 103.23) (end 183.94 102.8) (width 0.254) (layer "F.Cu") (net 5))
 (segment (start 185.51 102.8) (end 187.24 102.8) (width 0.254) (layer "F.Cu") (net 5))
 (segment (start 183.94 102.8) (end 185.51 102.8) (width 0.254) (layer "F.Cu") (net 5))
 (via (at 188.27 101.77) (size 0.8) (drill 0.4) (layers "F.Cu" "B.Cu") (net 5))
 (segment (start 188.27 101.77) (end 188.969999 101.070001) (width 0.254) (layer "B.Cu") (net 5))
 (segment (start 188.969999 101.070001) (end 191.550001 101.070001) (width 0.254) (layer "B.Cu") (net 5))
 (segment (start 190.96 102.98) (end 193.87 102.98) (width 0.254) (layer "F.Cu") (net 2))
 (segment (start 186.550001 98.570001) (end 190.96 102.98) (width 0.254) (layer "F.Cu") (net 2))
 (segment (start 193.87 102.98) (end 195.96 105.07) (width 0.254) (layer "F.Cu") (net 2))
 (segment (start 194.03 102.52) (end 195.95 102.52) (width 0.254) (layer "F.Cu") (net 1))
 (segment (start 191.550001 98.570001) (end 193.28 100.3) (width 0.254) (layer "F.Cu") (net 1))
 (segment (start 193.28 101.77) (end 194.03 102.52) (width 0.254) (layer "F.Cu") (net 1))
 (segment (start 193.28 100.3) (end 193.28 101.77) (width 0.254) (layer "F.Cu") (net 1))
 (segment (start 195.95 102.52) (end 198.5 105.07) (width 0.254) (layer "F.Cu") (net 1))
 (segment (start 180.500003 103.619997) (end 181.88 102.24) (width 0.254) (layer "F.Cu") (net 4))
 (segment (start 181.88 102.24) (end 185.380002 102.24) (width 0.254) (layer "F.Cu") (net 4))
 (segment (start 180.500003 105.070001) (end 180.500003 103.619997) (width 0.254) (layer "F.Cu") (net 4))
 (segment (start 185.380002 102.24) (end 186.550001 101.070001) (width 0.254) (layer "F.Cu") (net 4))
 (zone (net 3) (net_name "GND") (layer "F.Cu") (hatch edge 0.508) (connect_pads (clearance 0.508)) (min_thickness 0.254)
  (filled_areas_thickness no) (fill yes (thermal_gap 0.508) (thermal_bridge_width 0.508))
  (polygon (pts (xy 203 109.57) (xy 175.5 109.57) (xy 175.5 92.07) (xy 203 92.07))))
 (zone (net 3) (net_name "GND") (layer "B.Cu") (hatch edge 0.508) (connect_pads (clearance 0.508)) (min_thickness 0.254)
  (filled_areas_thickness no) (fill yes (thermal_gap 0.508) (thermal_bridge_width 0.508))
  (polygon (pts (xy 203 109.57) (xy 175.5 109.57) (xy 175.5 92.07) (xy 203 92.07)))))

